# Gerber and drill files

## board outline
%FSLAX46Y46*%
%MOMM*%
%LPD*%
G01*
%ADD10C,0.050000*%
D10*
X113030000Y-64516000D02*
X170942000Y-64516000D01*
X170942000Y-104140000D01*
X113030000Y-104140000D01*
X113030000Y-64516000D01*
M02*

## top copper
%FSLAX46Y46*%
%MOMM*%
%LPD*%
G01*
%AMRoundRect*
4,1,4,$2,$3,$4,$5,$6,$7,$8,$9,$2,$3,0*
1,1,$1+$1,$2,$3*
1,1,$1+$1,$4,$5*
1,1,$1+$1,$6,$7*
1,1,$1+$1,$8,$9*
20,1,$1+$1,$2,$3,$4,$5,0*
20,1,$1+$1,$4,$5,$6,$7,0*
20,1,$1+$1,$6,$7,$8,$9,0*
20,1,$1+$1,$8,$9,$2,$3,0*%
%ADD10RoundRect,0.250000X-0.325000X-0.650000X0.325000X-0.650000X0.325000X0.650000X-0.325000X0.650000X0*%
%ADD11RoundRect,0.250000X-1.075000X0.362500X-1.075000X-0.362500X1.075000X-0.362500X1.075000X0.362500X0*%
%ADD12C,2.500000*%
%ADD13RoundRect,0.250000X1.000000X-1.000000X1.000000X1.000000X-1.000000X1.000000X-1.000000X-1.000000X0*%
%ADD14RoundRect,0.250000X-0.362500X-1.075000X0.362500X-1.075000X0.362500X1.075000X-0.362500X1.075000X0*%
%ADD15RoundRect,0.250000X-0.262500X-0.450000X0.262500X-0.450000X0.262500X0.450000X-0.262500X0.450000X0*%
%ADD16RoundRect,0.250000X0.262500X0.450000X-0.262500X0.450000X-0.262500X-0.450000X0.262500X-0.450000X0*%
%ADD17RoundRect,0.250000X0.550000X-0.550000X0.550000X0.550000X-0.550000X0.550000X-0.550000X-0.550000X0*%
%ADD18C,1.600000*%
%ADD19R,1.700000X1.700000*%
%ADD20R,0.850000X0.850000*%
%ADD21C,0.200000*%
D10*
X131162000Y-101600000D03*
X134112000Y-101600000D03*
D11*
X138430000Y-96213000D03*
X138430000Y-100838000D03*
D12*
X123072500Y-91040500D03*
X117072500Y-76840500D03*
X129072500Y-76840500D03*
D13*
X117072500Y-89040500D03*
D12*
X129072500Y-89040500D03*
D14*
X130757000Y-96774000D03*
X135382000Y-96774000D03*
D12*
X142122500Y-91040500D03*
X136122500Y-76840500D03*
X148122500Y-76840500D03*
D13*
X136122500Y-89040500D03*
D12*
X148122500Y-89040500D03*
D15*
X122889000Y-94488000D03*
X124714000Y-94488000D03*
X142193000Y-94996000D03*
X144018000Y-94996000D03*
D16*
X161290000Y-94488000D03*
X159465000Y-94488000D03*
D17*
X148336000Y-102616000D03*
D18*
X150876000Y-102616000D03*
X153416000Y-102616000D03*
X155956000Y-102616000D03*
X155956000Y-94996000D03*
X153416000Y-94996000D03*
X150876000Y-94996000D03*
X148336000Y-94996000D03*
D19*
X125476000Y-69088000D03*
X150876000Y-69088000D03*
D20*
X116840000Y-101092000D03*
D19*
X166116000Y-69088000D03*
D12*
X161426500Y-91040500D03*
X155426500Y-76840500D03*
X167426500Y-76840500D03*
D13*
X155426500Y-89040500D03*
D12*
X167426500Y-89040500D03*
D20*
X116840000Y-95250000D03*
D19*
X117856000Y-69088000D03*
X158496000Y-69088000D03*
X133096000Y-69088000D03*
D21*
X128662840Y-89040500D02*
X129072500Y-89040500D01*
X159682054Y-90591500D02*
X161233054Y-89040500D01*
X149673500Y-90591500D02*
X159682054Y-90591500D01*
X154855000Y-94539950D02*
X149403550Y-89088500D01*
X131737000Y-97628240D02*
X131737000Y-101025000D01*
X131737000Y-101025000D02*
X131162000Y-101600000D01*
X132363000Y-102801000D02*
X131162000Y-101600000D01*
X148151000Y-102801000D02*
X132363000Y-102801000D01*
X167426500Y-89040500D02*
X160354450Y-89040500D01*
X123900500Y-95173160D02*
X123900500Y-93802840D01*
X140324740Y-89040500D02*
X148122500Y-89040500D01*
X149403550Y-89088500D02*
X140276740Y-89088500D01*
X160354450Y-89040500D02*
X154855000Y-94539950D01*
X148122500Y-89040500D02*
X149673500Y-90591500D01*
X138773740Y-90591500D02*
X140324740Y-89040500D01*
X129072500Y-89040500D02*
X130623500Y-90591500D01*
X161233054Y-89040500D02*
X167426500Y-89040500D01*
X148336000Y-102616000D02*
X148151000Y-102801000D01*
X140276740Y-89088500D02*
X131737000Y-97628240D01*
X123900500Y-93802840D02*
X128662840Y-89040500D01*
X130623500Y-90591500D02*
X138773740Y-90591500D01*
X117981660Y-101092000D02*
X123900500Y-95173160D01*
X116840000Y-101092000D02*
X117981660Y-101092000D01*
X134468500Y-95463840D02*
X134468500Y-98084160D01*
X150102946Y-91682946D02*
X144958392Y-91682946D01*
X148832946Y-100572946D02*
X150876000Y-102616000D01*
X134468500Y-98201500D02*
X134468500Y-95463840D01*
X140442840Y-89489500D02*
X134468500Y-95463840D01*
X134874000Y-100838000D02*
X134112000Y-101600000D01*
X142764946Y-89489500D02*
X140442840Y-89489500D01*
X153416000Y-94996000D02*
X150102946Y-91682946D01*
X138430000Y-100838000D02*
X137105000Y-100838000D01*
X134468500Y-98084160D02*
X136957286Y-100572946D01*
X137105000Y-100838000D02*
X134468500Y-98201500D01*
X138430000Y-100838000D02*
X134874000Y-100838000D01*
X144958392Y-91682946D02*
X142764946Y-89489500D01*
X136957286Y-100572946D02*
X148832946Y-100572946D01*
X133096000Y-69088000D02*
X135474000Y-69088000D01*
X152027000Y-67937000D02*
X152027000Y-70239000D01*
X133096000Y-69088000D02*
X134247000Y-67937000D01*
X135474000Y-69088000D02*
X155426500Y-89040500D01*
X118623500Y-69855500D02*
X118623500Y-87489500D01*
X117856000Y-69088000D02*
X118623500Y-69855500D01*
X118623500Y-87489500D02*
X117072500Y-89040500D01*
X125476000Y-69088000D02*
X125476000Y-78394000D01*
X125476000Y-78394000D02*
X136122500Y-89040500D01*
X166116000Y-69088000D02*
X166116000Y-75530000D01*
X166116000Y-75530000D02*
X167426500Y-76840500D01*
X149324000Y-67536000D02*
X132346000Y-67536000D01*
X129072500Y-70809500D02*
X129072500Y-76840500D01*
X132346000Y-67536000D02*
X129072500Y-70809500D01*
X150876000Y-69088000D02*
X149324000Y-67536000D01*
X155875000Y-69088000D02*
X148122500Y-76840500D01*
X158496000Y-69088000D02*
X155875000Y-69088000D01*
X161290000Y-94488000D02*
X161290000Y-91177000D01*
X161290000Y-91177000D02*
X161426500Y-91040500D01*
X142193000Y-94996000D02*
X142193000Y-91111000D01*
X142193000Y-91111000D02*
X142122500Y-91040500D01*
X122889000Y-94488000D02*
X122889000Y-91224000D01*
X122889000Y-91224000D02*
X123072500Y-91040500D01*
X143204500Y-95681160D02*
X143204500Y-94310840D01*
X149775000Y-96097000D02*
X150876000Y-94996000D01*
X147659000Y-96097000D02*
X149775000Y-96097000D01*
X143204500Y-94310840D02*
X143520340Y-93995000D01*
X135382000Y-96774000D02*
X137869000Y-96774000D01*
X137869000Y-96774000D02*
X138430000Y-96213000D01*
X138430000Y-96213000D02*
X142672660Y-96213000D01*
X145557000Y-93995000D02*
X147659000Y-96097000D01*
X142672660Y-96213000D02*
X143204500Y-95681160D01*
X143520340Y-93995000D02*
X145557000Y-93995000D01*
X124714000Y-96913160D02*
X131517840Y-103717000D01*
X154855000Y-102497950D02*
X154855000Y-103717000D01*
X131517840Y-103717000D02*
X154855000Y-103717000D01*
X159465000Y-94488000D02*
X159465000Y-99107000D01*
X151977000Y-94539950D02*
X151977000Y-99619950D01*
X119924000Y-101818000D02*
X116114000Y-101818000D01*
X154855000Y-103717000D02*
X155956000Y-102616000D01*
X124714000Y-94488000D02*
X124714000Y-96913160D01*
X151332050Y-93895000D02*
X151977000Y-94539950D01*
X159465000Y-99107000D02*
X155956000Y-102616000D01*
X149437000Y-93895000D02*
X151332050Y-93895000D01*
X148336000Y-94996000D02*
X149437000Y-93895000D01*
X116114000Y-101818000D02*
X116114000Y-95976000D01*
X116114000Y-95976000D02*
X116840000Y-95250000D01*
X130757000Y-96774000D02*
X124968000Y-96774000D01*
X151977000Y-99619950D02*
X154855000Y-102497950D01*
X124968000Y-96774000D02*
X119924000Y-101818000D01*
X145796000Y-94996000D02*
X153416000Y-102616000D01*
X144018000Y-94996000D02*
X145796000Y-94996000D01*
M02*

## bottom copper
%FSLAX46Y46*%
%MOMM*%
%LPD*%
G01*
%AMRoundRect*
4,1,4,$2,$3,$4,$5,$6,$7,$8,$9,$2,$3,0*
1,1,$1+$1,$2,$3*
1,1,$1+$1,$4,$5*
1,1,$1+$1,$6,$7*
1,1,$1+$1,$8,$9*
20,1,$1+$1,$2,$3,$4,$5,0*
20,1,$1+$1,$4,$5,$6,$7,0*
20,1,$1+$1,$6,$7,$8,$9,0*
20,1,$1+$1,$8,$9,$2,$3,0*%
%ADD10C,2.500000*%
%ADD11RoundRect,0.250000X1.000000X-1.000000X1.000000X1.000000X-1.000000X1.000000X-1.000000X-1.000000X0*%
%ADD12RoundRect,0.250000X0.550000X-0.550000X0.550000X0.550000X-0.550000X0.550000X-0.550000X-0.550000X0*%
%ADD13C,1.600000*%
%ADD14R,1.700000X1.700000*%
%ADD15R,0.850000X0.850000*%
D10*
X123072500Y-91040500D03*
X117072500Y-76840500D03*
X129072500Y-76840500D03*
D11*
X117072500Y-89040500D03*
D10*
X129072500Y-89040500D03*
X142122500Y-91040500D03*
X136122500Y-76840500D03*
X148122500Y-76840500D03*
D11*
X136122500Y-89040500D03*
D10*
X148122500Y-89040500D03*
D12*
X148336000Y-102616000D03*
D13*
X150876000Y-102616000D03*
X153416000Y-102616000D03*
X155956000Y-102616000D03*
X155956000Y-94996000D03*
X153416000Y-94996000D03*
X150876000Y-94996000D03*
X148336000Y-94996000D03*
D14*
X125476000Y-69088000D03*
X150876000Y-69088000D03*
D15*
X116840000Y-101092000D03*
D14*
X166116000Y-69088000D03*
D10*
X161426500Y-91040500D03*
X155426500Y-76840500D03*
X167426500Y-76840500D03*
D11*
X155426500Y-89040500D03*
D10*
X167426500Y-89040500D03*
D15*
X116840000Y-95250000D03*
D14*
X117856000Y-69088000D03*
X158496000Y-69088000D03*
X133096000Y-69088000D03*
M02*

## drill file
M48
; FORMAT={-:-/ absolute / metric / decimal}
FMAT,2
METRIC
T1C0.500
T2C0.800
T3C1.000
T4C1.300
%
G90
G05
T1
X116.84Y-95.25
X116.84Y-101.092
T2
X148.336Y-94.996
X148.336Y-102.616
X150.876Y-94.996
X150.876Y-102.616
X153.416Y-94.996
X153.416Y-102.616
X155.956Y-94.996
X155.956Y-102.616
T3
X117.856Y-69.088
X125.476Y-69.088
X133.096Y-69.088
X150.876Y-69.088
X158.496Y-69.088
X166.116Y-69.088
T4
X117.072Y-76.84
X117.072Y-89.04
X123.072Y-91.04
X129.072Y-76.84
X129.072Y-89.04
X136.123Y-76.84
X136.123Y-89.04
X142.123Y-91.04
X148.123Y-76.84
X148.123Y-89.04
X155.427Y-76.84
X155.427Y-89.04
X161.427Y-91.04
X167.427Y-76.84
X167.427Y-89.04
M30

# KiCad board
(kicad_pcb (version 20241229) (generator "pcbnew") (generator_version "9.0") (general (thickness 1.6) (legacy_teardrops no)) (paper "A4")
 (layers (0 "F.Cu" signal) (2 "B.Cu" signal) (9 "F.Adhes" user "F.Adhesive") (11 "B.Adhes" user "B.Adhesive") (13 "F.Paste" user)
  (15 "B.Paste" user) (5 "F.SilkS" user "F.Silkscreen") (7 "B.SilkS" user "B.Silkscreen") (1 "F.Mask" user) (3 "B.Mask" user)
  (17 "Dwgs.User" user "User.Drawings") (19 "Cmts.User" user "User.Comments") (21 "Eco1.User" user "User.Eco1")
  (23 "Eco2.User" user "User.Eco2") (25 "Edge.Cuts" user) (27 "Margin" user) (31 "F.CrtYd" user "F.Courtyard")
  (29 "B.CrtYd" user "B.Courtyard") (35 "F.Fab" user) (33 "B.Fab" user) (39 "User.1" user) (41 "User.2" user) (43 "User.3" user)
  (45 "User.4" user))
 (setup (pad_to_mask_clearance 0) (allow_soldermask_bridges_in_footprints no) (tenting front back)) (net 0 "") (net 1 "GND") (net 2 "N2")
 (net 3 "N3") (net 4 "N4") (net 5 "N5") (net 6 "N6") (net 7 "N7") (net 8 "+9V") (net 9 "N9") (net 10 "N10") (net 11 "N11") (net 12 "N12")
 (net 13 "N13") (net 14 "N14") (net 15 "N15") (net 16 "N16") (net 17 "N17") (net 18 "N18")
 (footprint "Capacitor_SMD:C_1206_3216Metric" (layer "F.Cu") (at 132.637 101.6)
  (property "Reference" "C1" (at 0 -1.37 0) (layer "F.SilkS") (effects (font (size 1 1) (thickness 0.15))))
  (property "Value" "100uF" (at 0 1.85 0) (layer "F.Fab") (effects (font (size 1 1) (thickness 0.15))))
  (pad "1" smd roundrect (at -1.475 0) (size 1.15 1.8) (layers "F.Cu" "F.Mask" "F.Paste") (roundrect_rratio 0.217391) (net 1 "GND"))
  (pad "2" smd roundrect (at 1.475 0) (size 1.15 1.8) (layers "F.Cu" "F.Mask" "F.Paste") (roundrect_rratio 0.217391) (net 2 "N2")))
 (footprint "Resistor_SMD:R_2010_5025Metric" (layer "F.Cu") (at 138.43 98.5255 -90)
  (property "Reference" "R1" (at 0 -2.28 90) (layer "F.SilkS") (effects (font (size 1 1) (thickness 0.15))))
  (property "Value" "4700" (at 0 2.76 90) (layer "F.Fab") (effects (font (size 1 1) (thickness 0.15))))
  (pad "1" smd roundrect (at -2.3125 0 270) (size 1.225 2.65) (layers "F.Cu" "F.Mask" "F.Paste") (roundrect_rratio 0.204082) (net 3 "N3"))
  (pad "2" smd roundrect (at 2.3125 0 270) (size 1.225 2.65) (layers "F.Cu" "F.Mask" "F.Paste") (roundrect_rratio 0.204082) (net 2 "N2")))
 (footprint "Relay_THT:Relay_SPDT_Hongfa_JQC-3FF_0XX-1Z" (layer "F.Cu") (at 117.0725 89.0405 90)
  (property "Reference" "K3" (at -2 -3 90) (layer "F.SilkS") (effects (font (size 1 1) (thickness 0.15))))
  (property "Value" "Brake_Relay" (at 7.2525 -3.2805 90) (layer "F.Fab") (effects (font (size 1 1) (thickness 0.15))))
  (pad "11" thru_hole circle (at -2 6 90) (size 2.5 2.5) (drill 1.3) (layers "*.Cu" "*.Mask") (remove_unused_layers no) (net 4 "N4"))
  (pad "12" thru_hole circle (at 12.2 0 90) (size 2.5 2.5) (drill 1.3) (layers "*.Cu" "*.Mask") (remove_unused_layers no) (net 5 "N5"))
  (pad "14" thru_hole circle (at 12.2 12 90) (size 2.5 2.5) (drill 1.3) (layers "*.Cu" "*.Mask") (remove_unused_layers no) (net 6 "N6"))
  (pad "A1" thru_hole roundrect (at 0 0 90) (size 2.5 2.5) (drill 1.3) (layers "*.Cu" "*.Mask") (remove_unused_layers no)
   (roundrect_rratio 0.1) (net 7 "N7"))
  (pad "A2" thru_hole circle (at 0 12 90) (size 2.5 2.5) (drill 1.3) (layers "*.Cu" "*.Mask") (remove_unused_layers no) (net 1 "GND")))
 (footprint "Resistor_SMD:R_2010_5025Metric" (layer "F.Cu") (at 133.0695 96.774)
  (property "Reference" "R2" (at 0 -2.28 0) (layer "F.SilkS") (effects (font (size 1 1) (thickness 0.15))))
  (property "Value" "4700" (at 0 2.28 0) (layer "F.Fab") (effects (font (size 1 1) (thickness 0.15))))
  (pad "1" smd roundrect (at -2.3125 0) (size 1.225 2.65) (layers "F.Cu" "F.Mask" "F.Paste") (roundrect_rratio 0.204082) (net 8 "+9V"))
  (pad "2" smd roundrect (at 2.3125 0) (size 1.225 2.65) (layers "F.Cu" "F.Mask" "F.Paste") (roundrect_rratio 0.204082) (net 3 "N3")))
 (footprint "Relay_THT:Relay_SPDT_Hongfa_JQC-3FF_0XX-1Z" (layer "F.Cu") (at 136.1225 89.0405 90)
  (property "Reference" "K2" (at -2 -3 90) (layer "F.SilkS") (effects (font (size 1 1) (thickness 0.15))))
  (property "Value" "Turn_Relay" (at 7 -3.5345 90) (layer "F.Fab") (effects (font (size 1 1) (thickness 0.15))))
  (pad "11" thru_hole circle (at -2 6 90) (size 2.5 2.5) (drill 1.3) (layers "*.Cu" "*.Mask") (remove_unused_layers no) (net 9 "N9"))
  (pad "12" thru_hole circle (at 12.2 0 90) (size 2.5 2.5) (drill 1.3) (layers "*.Cu" "*.Mask") (remove_unused_layers no) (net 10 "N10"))
  (pad "14" thru_hole circle (at 12.2 12 90) (size 2.5 2.5) (drill 1.3) (layers "*.Cu" "*.Mask") (remove_unused_layers no) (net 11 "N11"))
  (pad "A1" thru_hole roundrect (at 0 0 90) (size 2.5 2.5) (drill 1.3) (layers "*.Cu" "*.Mask") (remove_unused_layers no)
   (roundrect_rratio 0.1) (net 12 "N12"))
  (pad "A2" thru_hole circle (at 0 12 90) (size 2.5 2.5) (drill 1.3) (layers "*.Cu" "*.Mask") (remove_unused_layers no) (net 1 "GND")))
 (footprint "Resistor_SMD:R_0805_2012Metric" (layer "F.Cu") (at 123.8015 94.488)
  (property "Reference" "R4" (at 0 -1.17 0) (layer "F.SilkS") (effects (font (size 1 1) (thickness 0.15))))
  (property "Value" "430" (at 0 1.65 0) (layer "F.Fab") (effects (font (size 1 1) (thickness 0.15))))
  (pad "1" smd roundrect (at -0.9125 0) (size 1.025 1.4) (layers "F.Cu" "F.Mask" "F.Paste") (roundrect_rratio 0.243902) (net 4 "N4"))
  (pad "2" smd roundrect (at 0.9125 0) (size 1.025 1.4) (layers "F.Cu" "F.Mask" "F.Paste") (roundrect_rratio 0.243902) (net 8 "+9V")))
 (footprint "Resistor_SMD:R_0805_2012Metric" (layer "F.Cu") (at 143.1055 94.996)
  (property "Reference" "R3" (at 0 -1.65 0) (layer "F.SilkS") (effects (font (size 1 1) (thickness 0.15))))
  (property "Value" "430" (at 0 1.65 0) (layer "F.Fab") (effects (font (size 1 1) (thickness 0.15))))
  (pad "1" smd roundrect (at -0.9125 0) (size 1.025 1.4) (layers "F.Cu" "F.Mask" "F.Paste") (roundrect_rratio 0.243902) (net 9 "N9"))
  (pad "2" smd roundrect (at 0.9125 0) (size 1.025 1.4) (layers "F.Cu" "F.Mask" "F.Paste") (roundrect_rratio 0.243902) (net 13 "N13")))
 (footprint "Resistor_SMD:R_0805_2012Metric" (layer "F.Cu") (at 160.3775 94.488 180)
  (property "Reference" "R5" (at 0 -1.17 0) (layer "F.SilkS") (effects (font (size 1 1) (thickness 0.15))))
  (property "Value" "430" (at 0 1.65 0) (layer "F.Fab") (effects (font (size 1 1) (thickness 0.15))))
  (pad "1" smd roundrect (at -0.9125 0 180) (size 1.025 1.4) (layers "F.Cu" "F.Mask" "F.Paste") (roundrect_rratio 0.243902) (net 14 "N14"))
  (pad "2" smd roundrect (at 0.9125 0 180) (size 1.025 1.4) (layers "F.Cu" "F.Mask" "F.Paste") (roundrect_rratio 0.243902) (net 8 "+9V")))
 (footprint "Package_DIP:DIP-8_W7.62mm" (layer "F.Cu") (at 148.336 102.616 90)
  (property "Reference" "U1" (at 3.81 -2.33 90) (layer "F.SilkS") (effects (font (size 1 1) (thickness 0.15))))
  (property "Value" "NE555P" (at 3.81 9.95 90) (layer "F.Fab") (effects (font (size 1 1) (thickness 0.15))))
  (pad "1" thru_hole roundrect (at 0 0 90) (size 1.6 1.6) (drill 0.8) (layers "*.Cu" "*.Mask") (remove_unused_layers no)
   (roundrect_rratio 0.15625) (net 1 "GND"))
  (pad "2" thru_hole circle (at 0 2.54 90) (size 1.6 1.6) (drill 0.8) (layers "*.Cu" "*.Mask") (remove_unused_layers no) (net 2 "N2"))
  (pad "3" thru_hole circle (at 0 5.08 90) (size 1.6 1.6) (drill 0.8) (layers "*.Cu" "*.Mask") (remove_unused_layers no) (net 13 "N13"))
  (pad "4" thru_hole circle (at 0 7.62 90) (size 1.6 1.6) (drill 0.8) (layers "*.Cu" "*.Mask") (remove_unused_layers no) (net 8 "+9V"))
  (pad "5" thru_hole circle (at 7.62 7.62 90) (size 1.6 1.6) (drill 0.8) (layers "*.Cu" "*.Mask") (remove_unused_layers no) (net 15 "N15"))
  (pad "6" thru_hole circle (at 7.62 5.08 90) (size 1.6 1.6) (drill 0.8) (layers "*.Cu" "*.Mask") (remove_unused_layers no) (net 2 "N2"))
  (pad "7" thru_hole circle (at 7.62 2.54 90) (size 1.6 1.6) (drill 0.8) (layers "*.Cu" "*.Mask") (remove_unused_layers no) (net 3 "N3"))
  (pad "8" thru_hole circle (at 7.62 0 90) (size 1.6 1.6) (drill 0.8) (layers "*.Cu" "*.Mask") (remove_unused_layers no) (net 8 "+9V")))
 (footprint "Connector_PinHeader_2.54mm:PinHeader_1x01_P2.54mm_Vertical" (layer "F.Cu") (at 125.476 69.088 -90)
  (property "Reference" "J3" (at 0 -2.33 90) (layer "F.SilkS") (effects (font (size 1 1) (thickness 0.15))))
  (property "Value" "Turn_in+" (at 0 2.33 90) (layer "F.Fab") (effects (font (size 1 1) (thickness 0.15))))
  (pad "1" thru_hole rect (at 0 0 270) (size 1.7 1.7) (drill 1) (layers "*.Cu" "*.Mask") (remove_unused_layers no) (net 12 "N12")))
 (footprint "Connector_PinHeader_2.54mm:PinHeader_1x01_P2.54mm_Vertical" (layer "F.Cu") (at 150.876 69.088 -90)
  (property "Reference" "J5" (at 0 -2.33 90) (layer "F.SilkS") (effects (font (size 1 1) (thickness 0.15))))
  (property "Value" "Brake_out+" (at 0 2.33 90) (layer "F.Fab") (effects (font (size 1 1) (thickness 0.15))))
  (pad "1" thru_hole rect (at 0 0 270) (size 1.7 1.7) (drill 1) (layers "*.Cu" "*.Mask") (remove_unused_layers no) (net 6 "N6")))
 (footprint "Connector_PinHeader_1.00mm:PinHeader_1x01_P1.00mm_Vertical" (layer "F.Cu") (at 116.84 101.092)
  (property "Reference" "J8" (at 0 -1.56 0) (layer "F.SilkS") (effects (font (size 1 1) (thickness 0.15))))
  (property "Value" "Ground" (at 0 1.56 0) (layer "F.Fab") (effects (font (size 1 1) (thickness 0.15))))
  (pad "1" thru_hole rect (at 0 0) (size 0.85 0.85) (drill 0.5) (layers "*.Cu" "*.Mask") (remove_unused_layers no) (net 1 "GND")))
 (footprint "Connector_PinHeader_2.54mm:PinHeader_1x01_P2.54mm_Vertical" (layer "F.Cu") (at 166.116 69.088 -90)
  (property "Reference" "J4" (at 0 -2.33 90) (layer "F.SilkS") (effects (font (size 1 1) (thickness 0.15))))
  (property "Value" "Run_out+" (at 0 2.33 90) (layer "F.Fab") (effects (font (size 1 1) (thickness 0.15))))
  (pad "1" thru_hole rect (at 0 0 270) (size 1.7 1.7) (drill 1) (layers "*.Cu" "*.Mask") (remove_unused_layers no) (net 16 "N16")))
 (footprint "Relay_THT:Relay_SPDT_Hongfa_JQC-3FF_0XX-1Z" (layer "F.Cu") (at 155.4265 89.0405 90)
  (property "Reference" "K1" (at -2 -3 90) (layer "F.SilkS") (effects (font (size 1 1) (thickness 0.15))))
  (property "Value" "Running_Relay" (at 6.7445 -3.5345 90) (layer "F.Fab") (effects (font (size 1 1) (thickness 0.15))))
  (pad "11" thru_hole circle (at -2 6 90) (size 2.5 2.5) (drill 1.3) (layers "*.Cu" "*.Mask") (remove_unused_layers no) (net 14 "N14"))
  (pad "12" thru_hole circle (at 12.2 0 90) (size 2.5 2.5) (drill 1.3) (layers "*.Cu" "*.Mask") (remove_unused_layers no) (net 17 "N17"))
  (pad "14" thru_hole circle (at 12.2 12 90) (size 2.5 2.5) (drill 1.3) (layers "*.Cu" "*.Mask") (remove_unused_layers no) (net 16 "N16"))
  (pad "A1" thru_hole roundrect (at 0 0 90) (size 2.5 2.5) (drill 1.3) (layers "*.Cu" "*.Mask") (remove_unused_layers no)
   (roundrect_rratio 0.1) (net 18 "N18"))
  (pad "A2" thru_hole circle (at 0 12 90) (size 2.5 2.5) (drill 1.3) (layers "*.Cu" "*.Mask") (remove_unused_layers no) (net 1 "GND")))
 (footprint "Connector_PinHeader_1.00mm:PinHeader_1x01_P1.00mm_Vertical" (layer "F.Cu") (at 116.84 95.25)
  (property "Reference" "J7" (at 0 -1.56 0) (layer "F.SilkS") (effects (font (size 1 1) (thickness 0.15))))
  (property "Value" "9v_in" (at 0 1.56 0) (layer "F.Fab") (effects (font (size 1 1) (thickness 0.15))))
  (pad "1" thru_hole rect (at 0 0) (size 0.85 0.85) (drill 0.5) (layers "*.Cu" "*.Mask") (remove_unused_layers no) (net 8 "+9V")))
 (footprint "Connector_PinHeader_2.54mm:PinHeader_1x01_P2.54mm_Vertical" (layer "F.Cu") (at 117.856 69.088 -90)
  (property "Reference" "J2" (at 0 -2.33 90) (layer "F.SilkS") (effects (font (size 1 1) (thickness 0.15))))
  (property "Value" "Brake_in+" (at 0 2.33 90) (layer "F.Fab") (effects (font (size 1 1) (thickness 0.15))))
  (pad "1" thru_hole rect (at 0 0 270) (size 1.7 1.7) (drill 1) (layers "*.Cu" "*.Mask") (remove_unused_layers no) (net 7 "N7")))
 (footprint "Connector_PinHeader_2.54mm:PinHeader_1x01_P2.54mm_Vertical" (layer "F.Cu") (at 158.496 69.088 -90)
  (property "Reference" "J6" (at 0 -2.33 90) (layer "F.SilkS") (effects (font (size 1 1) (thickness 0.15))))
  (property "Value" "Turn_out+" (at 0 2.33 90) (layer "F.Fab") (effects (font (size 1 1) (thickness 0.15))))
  (pad "1" thru_hole rect (at 0 0 270) (size 1.7 1.7) (drill 1) (layers "*.Cu" "*.Mask") (remove_unused_layers no) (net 11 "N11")))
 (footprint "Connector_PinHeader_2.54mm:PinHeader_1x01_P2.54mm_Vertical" (layer "F.Cu") (at 133.096 69.088 -90)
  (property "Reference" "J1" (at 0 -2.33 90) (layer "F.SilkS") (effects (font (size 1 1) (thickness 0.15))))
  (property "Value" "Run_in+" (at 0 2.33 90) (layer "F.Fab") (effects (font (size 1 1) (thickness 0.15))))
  (pad "1" thru_hole rect (at 0 0 270) (size 1.7 1.7) (drill 1) (layers "*.Cu" "*.Mask") (remove_unused_layers no) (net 18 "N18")))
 (gr_rect (start 113.03 64.516) (end 170.942 104.14) (stroke (width 0.05) (type default)) (fill no) (layer "Edge.Cuts"))
 (segment (start 128.66284 89.0405) (end 129.0725 89.0405) (width 0.2) (layer "F.Cu") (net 1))
 (segment (start 159.682054 90.5915) (end 161.233054 89.0405) (width 0.2) (layer "F.Cu") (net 1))
 (segment (start 149.6735 90.5915) (end 159.682054 90.5915) (width 0.2) (layer "F.Cu") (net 1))
 (segment (start 154.855 94.53995) (end 149.40355 89.0885) (width 0.2) (layer "F.Cu") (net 1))
 (segment (start 131.737 97.62824) (end 131.737 101.025) (width 0.2) (layer "F.Cu") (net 1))
 (segment (start 131.737 101.025) (end 131.162 101.6) (width 0.2) (layer "F.Cu") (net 1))
 (segment (start 132.363 102.801) (end 131.162 101.6) (width 0.2) (layer "F.Cu") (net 1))
 (segment (start 148.151 102.801) (end 132.363 102.801) (width 0.2) (layer "F.Cu") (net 1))
 (segment (start 167.4265 89.0405) (end 160.35445 89.0405) (width 0.2) (layer "F.Cu") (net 1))
 (segment (start 123.9005 95.17316) (end 123.9005 93.80284) (width 0.2) (layer "F.Cu") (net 1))
 (segment (start 140.32474 89.0405) (end 148.1225 89.0405) (width 0.2) (layer "F.Cu") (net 1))
 (segment (start 149.40355 89.0885) (end 140.27674 89.0885) (width 0.2) (layer "F.Cu") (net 1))
 (segment (start 160.35445 89.0405) (end 154.855 94.53995) (width 0.2) (layer "F.Cu") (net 1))
 (segment (start 148.1225 89.0405) (end 149.6735 90.5915) (width 0.2) (layer "F.Cu") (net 1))
 (segment (start 138.77374 90.5915) (end 140.32474 89.0405) (width 0.2) (layer "F.Cu") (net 1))
 (segment (start 129.0725 89.0405) (end 130.6235 90.5915) (width 0.2) (layer "F.Cu") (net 1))
 (segment (start 161.233054 89.0405) (end 167.4265 89.0405) (width 0.2) (layer "F.Cu") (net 1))
 (segment (start 148.336 102.616) (end 148.151 102.801) (width 0.2) (layer "F.Cu") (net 1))
 (segment (start 140.27674 89.0885) (end 131.737 97.62824) (width 0.2) (layer "F.Cu") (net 1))
 (segment (start 123.9005 93.80284) (end 128.66284 89.0405) (width 0.2) (layer "F.Cu") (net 1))
 (segment (start 130.6235 90.5915) (end 138.77374 90.5915) (width 0.2) (layer "F.Cu") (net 1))
 (segment (start 117.98166 101.092) (end 123.9005 95.17316) (width 0.2) (layer "F.Cu") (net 1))
 (segment (start 116.84 101.092) (end 117.98166 101.092) (width 0.2) (layer "F.Cu") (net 1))
 (segment (start 134.4685 95.46384) (end 134.4685 98.08416) (width 0.2) (layer "F.Cu") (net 2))
 (segment (start 150.102946 91.682946) (end 144.958392 91.682946) (width 0.2) (layer "F.Cu") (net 2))
 (segment (start 148.832946 100.572946) (end 150.876 102.616) (width 0.2) (layer "F.Cu") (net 2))
 (segment (start 134.4685 98.2015) (end 134.4685 95.46384) (width 0.2) (layer "F.Cu") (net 2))
 (segment (start 140.44284 89.4895) (end 134.4685 95.46384) (width 0.2) (layer "F.Cu") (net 2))
 (segment (start 134.874 100.838) (end 134.112 101.6) (width 0.2) (layer "F.Cu") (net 2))
 (segment (start 142.764946 89.4895) (end 140.44284 89.4895) (width 0.2) (layer "F.Cu") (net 2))
 (segment (start 153.416 94.996) (end 150.102946 91.682946) (width 0.2) (layer "F.Cu") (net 2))
 (segment (start 138.43 100.838) (end 137.105 100.838) (width 0.2) (layer "F.Cu") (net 2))
 (segment (start 134.4685 98.08416) (end 136.957286 100.572946) (width 0.2) (layer "F.Cu") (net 2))
 (segment (start 137.105 100.838) (end 134.4685 98.2015) (width 0.2) (layer "F.Cu") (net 2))
 (segment (start 138.43 100.838) (end 134.874 100.838) (width 0.2) (layer "F.Cu") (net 2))
 (segment (start 144.958392 91.682946) (end 142.764946 89.4895) (width 0.2) (layer "F.Cu") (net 2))
 (segment (start 136.957286 100.572946) (end 148.832946 100.572946) (width 0.2) (layer "F.Cu") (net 2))
 (segment (start 133.096 69.088) (end 135.474 69.088) (width 0.2) (layer "F.Cu") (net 18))
 (segment (start 152.027 67.937) (end 152.027 70.239) (width 0.2) (layer "F.Cu") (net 18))
 (segment (start 133.096 69.088) (end 134.247 67.937) (width 0.2) (layer "F.Cu") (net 18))
 (segment (start 135.474 69.088) (end 155.4265 89.0405) (width 0.2) (layer "F.Cu") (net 18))
 (segment (start 118.6235 69.8555) (end 118.6235 87.4895) (width 0.2) (layer "F.Cu") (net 7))
 (segment (start 117.856 69.088) (end 118.6235 69.8555) (width 0.2) (layer "F.Cu") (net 7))
 (segment (start 118.6235 87.4895) (end 117.0725 89.0405) (width 0.2) (layer "F.Cu") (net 7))
 (segment (start 125.476 69.088) (end 125.476 78.394) (width 0.2) (layer "F.Cu") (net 12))
 (segment (start 125.476 78.394) (end 136.1225 89.0405) (width 0.2) (layer "F.Cu") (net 12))
 (segment (start 166.116 69.088) (end 166.116 75.53) (width 0.2) (layer "F.Cu") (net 16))
 (segment (start 166.116 75.53) (end 167.4265 76.8405) (width 0.2) (layer "F.Cu") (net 16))
 (segment (start 149.324 67.536) (end 132.346 67.536) (width 0.2) (layer "F.Cu") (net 6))
 (segment (start 129.0725 70.8095) (end 129.0725 76.8405) (width 0.2) (layer "F.Cu") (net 6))
 (segment (start 132.346 67.536) (end 129.0725 70.8095) (width 0.2) (layer "F.Cu") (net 6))
 (segment (start 150.876 69.088) (end 149.324 67.536) (width 0.2) (layer "F.Cu") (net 6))
 (segment (start 155.875 69.088) (end 148.1225 76.8405) (width 0.2) (layer "F.Cu") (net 11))
 (segment (start 158.496 69.088) (end 155.875 69.088) (width 0.2) (layer "F.Cu") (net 11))
 (segment (start 161.29 94.488) (end 161.29 91.177) (width 0.2) (layer "F.Cu") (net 14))
 (segment (start 161.29 91.177) (end 161.4265 91.0405) (width 0.2) (layer "F.Cu") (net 14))
 (segment (start 142.193 94.996) (end 142.193 91.111) (width 0.2) (layer "F.Cu") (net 9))
 (segment (start 142.193 91.111) (end 142.1225 91.0405) (width 0.2) (layer "F.Cu") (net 9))
 (segment (start 122.889 94.488) (end 122.889 91.224) (width 0.2) (layer "F.Cu") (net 4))
 (segment (start 122.889 91.224) (end 123.0725 91.0405) (width 0.2) (layer "F.Cu") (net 4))
 (segment (start 143.2045 95.68116) (end 143.2045 94.31084) (width 0.2) (layer "F.Cu") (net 3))
 (segment (start 149.775 96.097) (end 150.876 94.996) (width 0.2) (layer "F.Cu") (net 3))
 (segment (start 147.659 96.097) (end 149.775 96.097) (width 0.2) (layer "F.Cu") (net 3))
 (segment (start 143.2045 94.31084) (end 143.52034 93.995) (width 0.2) (layer "F.Cu") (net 3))
 (segment (start 135.382 96.774) (end 137.869 96.774) (width 0.2) (layer "F.Cu") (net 3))
 (segment (start 137.869 96.774) (end 138.43 96.213) (width 0.2) (layer "F.Cu") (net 3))
 (segment (start 138.43 96.213) (end 142.67266 96.213) (width 0.2) (layer "F.Cu") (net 3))
 (segment (start 145.557 93.995) (end 147.659 96.097) (width 0.2) (layer "F.Cu") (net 3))
 (segment (start 142.67266 96.213) (end 143.2045 95.68116) (width 0.2) (layer "F.Cu") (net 3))
 (segment (start 143.52034 93.995) (end 145.557 93.995) (width 0.2) (layer "F.Cu") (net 3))
 (segment (start 124.714 96.91316) (end 131.51784 103.717) (width 0.2) (layer "F.Cu") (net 8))
 (segment (start 154.855 102.49795) (end 154.855 103.717) (width 0.2) (layer "F.Cu") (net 8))
 (segment (start 131.51784 103.717) (end 154.855 103.717) (width 0.2) (layer "F.Cu") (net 8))
 (segment (start 159.465 94.488) (end 159.465 99.107) (width 0.2) (layer "F.Cu") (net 8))
 (segment (start 151.977 94.53995) (end 151.977 99.61995) (width 0.2) (layer "F.Cu") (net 8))
 (segment (start 119.924 101.818) (end 116.114 101.818) (width 0.2) (layer "F.Cu") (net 8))
 (segment (start 154.855 103.717) (end 155.956 102.616) (width 0.2) (layer "F.Cu") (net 8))
 (segment (start 124.714 94.488) (end 124.714 96.91316) (width 0.2) (layer "F.Cu") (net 8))
 (segment (start 151.33205 93.895) (end 151.977 94.53995) (width 0.2) (layer "F.Cu") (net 8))
 (segment (start 159.465 99.107) (end 155.956 102.616) (width 0.2) (layer "F.Cu") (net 8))
 (segment (start 149.437 93.895) (end 151.33205 93.895) (width 0.2) (layer "F.Cu") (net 8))
 (segment (start 148.336 94.996) (end 149.437 93.895) (width 0.2) (layer "F.Cu") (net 8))
 (segment (start 116.114 101.818) (end 116.114 95.976) (width 0.2) (layer "F.Cu") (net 8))
 (segment (start 116.114 95.976) (end 116.84 95.25) (width 0.2) (layer "F.Cu") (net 8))
 (segment (start 130.757 96.774) (end 124.968 96.774) (width 0.2) (layer "F.Cu") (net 8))
 (segment (start 151.977 99.61995) (end 154.855 102.49795) (width 0.2) (layer "F.Cu") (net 8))
 (segment (start 124.968 96.774) (end 119.924 101.818) (width 0.2) (layer "F.Cu") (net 8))
 (segment (start 145.796 94.996) (end 153.416 102.616) (width 0.2) (layer "F.Cu") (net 13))
 (segment (start 144.018 94.996) (end 145.796 94.996) (width 0.2) (layer "F.Cu") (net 13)))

